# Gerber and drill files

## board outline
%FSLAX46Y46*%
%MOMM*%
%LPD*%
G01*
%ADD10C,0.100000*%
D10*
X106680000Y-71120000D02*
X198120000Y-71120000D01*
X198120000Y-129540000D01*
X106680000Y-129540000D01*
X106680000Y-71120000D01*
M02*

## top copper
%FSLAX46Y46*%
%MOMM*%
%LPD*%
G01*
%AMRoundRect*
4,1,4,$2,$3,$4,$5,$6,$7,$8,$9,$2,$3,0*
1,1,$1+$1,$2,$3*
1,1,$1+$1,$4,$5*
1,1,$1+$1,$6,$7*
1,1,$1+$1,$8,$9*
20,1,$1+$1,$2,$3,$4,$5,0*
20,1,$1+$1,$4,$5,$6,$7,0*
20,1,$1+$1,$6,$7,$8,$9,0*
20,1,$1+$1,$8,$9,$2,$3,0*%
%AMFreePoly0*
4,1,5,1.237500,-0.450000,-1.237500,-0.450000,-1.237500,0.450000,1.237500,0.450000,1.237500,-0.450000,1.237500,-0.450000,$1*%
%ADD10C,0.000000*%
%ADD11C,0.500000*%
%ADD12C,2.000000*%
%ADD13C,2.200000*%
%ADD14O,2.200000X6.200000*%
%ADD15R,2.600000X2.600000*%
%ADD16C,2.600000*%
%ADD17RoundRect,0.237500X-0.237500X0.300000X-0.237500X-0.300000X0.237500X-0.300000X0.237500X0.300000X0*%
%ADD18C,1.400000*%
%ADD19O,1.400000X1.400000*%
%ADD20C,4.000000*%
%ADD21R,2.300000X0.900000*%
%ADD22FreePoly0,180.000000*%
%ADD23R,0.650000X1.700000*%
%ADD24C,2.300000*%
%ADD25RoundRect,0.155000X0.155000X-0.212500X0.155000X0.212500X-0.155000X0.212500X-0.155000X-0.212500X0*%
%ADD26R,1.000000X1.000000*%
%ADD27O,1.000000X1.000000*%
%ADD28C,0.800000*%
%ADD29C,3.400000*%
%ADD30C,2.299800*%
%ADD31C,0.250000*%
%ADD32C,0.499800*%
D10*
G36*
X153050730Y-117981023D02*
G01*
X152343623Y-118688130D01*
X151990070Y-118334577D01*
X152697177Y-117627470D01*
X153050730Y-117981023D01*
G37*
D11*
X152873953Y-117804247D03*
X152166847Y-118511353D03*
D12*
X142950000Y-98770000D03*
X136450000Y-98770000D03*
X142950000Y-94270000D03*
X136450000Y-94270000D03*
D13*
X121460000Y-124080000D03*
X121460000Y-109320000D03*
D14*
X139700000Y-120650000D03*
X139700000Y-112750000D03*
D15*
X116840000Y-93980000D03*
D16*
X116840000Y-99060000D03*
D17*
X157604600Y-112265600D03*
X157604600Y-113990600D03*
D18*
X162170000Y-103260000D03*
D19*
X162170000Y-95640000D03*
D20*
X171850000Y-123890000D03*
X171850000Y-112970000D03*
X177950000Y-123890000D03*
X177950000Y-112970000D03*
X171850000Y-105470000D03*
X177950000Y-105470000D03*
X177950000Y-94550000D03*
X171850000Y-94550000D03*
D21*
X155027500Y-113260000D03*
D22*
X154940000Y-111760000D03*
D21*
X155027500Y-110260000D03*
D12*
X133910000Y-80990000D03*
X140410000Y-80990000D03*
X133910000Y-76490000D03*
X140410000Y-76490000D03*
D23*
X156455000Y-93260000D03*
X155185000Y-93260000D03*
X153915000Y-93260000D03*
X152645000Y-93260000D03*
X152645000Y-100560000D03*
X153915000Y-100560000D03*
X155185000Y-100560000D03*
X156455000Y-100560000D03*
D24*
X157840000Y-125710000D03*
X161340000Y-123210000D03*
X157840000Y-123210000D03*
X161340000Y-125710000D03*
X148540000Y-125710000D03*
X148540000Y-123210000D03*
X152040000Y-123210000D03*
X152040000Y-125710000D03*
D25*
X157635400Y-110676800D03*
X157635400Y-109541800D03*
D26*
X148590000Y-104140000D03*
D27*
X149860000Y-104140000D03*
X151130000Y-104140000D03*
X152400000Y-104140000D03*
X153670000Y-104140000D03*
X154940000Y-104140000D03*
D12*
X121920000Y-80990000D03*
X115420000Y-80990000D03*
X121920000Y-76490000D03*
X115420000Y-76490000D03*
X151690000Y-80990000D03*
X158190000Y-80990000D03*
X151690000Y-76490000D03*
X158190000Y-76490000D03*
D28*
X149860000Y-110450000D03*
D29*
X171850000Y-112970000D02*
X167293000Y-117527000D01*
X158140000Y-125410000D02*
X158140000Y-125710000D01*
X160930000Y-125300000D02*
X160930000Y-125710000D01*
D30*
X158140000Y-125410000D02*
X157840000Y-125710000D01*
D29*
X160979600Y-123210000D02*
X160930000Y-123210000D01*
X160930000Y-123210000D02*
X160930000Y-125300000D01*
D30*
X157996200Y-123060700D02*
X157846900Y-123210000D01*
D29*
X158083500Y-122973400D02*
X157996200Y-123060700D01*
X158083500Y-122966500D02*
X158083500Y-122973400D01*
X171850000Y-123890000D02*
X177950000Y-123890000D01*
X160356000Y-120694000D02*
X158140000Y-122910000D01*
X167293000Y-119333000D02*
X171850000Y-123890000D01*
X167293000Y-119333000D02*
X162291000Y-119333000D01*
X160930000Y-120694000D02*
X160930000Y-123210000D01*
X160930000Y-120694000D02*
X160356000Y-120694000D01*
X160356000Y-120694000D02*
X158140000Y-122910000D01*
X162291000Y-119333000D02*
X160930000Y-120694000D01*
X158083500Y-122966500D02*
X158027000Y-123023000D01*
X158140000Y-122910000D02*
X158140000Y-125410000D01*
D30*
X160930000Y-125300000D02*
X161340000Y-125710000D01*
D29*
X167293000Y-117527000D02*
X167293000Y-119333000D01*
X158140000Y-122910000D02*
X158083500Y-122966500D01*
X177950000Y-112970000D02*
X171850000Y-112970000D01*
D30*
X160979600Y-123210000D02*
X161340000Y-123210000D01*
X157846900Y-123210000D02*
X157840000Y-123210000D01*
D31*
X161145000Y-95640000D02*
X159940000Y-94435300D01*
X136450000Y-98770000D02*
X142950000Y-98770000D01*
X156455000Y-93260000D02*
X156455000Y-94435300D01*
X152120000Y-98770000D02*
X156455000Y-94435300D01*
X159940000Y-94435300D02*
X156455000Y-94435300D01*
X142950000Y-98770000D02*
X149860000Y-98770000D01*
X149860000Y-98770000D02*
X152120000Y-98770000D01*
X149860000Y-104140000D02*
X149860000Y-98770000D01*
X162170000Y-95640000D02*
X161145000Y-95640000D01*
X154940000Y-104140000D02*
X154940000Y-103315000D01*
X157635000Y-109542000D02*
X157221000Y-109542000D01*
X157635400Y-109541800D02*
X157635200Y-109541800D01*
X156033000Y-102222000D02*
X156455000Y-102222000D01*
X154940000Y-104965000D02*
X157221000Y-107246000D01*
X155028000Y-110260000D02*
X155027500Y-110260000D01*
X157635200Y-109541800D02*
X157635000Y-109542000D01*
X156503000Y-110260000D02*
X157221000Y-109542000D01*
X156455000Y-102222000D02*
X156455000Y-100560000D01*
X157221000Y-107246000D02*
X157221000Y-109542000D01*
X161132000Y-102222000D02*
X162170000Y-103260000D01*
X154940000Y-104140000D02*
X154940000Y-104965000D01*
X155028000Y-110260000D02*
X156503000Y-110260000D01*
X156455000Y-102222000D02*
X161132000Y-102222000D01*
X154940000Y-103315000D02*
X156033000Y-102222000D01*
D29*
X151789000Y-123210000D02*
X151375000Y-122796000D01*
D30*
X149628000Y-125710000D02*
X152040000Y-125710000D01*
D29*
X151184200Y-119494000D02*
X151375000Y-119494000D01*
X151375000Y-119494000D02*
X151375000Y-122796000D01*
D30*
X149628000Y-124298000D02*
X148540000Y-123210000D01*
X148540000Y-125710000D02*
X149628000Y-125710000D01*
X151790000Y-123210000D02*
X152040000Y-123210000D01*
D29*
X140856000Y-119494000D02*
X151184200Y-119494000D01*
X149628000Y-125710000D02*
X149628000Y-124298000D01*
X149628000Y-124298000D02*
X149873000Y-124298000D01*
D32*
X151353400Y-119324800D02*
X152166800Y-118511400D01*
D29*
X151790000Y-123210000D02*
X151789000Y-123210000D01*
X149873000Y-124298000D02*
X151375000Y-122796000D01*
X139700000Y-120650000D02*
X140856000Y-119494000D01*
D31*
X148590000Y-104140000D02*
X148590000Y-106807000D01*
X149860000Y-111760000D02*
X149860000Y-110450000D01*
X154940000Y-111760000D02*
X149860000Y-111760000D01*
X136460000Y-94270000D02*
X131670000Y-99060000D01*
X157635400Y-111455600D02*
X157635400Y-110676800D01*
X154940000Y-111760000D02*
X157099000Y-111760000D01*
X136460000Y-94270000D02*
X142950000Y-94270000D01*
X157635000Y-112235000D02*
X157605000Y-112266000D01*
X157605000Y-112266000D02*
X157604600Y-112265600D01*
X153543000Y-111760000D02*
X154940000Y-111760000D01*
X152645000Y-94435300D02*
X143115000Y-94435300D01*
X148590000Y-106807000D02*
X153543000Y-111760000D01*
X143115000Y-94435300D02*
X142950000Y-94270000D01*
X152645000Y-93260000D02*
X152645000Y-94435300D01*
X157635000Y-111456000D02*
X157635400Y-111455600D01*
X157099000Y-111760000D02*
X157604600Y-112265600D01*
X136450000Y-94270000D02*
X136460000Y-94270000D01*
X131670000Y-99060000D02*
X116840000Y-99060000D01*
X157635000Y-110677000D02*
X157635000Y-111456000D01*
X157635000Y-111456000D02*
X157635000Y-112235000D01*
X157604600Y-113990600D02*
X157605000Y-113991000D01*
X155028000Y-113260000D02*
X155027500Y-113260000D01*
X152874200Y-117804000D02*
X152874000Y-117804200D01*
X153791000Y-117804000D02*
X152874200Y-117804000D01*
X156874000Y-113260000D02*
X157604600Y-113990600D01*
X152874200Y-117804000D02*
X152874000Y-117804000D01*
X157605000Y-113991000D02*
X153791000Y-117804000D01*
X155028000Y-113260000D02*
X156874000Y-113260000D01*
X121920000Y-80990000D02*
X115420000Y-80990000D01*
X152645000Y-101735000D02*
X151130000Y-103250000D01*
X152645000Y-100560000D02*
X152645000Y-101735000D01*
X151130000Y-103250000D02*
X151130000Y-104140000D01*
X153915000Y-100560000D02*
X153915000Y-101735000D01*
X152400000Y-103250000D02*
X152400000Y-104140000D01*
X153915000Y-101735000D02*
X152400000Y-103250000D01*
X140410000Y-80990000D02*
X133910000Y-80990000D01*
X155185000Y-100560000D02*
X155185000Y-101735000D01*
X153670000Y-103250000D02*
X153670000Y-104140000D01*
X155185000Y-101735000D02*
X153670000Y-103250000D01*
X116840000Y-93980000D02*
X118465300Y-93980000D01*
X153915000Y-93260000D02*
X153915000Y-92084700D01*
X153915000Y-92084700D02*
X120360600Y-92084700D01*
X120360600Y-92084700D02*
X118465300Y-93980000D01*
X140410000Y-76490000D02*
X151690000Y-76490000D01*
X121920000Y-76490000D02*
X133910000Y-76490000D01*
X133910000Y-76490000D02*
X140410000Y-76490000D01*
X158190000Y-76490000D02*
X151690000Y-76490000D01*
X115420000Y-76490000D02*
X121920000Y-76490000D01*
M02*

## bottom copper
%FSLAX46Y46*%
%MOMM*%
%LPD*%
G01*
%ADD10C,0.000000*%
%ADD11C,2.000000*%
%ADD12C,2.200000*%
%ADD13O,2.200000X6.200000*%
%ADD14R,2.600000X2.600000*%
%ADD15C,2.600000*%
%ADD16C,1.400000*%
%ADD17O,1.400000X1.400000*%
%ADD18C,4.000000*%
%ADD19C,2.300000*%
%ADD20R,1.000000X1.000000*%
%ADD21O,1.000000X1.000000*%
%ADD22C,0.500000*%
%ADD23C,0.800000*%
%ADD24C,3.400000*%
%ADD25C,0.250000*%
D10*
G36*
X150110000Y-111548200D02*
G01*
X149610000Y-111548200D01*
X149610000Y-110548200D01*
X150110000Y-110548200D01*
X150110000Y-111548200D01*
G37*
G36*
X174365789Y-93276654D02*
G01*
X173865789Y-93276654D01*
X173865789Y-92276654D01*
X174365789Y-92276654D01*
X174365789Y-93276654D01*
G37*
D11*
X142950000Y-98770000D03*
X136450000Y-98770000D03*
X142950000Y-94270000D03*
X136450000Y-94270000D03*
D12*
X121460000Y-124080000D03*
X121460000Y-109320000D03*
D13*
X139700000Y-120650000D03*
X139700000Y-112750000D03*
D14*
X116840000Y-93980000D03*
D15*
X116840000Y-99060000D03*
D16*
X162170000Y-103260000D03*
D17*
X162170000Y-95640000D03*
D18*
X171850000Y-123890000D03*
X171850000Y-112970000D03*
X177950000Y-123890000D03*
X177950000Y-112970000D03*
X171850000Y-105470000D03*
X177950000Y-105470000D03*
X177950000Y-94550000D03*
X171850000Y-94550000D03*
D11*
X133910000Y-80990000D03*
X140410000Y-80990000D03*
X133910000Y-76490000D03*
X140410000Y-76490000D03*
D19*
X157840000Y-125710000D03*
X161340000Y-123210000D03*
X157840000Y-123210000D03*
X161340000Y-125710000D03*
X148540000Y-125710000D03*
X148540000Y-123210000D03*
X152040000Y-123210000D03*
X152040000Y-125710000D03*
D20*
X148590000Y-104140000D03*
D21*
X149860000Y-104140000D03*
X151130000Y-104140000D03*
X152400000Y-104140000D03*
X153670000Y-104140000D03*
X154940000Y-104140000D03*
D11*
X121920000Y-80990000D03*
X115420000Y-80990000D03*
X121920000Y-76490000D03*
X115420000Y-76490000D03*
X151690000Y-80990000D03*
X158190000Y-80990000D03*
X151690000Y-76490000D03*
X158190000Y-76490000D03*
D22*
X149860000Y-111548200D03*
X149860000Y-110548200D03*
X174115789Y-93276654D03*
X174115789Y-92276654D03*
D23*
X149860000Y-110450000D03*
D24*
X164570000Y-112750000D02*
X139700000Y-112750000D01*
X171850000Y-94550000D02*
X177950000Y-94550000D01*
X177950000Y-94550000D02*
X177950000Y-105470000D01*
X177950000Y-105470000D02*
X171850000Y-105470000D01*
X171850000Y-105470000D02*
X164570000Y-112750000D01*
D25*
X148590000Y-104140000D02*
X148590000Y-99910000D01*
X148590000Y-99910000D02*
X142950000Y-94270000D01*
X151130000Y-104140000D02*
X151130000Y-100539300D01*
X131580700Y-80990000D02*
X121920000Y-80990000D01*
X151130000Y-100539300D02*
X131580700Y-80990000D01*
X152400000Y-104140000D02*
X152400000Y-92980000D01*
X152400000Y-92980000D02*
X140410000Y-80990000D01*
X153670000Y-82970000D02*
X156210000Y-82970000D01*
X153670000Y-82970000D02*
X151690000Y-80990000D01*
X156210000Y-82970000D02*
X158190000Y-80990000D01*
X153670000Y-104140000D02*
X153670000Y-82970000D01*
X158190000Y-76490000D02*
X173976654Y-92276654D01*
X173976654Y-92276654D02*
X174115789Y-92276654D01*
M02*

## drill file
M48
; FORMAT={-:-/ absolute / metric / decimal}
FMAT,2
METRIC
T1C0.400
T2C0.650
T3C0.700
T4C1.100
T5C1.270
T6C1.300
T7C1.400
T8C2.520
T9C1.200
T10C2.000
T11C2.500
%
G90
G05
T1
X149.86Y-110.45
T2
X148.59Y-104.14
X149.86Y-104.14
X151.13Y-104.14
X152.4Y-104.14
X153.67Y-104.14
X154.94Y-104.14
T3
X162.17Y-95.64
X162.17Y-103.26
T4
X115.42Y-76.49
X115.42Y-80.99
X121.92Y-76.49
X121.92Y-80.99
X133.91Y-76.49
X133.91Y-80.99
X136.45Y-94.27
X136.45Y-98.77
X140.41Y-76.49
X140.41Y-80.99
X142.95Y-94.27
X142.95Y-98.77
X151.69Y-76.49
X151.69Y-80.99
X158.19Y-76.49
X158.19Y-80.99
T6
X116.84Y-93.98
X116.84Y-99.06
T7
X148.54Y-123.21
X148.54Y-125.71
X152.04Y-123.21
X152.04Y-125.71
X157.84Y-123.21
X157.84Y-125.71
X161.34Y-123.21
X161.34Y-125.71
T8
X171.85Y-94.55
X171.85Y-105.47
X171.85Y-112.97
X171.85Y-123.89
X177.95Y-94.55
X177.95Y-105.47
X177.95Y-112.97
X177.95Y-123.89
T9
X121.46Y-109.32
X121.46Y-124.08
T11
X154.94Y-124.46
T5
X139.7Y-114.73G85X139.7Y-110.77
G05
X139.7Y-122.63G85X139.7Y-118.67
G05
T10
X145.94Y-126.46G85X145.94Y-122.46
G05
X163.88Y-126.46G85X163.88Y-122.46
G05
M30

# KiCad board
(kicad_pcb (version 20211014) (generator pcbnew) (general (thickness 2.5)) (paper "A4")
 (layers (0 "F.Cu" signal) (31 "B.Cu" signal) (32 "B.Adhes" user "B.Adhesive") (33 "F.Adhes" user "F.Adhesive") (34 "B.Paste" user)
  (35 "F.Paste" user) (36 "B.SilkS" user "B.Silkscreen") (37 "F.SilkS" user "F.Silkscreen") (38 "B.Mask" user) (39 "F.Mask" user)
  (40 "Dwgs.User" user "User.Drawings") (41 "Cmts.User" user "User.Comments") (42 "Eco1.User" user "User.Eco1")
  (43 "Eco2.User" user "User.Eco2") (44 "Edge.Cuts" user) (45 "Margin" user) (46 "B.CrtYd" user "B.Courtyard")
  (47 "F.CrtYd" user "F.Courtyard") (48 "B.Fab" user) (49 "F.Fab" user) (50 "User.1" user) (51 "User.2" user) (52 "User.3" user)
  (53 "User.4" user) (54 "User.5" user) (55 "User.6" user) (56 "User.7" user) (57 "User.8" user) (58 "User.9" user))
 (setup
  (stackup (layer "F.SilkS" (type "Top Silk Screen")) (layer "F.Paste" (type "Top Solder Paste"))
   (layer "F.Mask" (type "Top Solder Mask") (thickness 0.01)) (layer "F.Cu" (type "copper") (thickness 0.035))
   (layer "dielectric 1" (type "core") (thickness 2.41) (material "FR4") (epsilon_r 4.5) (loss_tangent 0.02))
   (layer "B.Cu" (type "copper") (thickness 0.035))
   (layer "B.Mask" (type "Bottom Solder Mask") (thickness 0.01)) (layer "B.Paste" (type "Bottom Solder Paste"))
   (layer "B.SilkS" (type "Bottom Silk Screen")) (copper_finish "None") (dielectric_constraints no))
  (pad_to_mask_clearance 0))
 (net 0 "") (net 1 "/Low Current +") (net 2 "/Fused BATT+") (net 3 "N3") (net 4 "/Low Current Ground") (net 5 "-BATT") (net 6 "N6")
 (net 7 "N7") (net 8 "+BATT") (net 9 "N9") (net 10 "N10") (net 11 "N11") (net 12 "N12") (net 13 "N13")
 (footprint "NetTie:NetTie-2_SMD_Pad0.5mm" (layer "F.Cu") (at 152.5204 118.1578 -135)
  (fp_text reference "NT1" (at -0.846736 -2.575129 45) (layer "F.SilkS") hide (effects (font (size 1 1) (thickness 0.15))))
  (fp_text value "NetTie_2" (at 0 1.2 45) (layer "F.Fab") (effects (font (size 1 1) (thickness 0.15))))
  (fp_poly (pts (xy -0.5 -0.25) (xy 0.5 -0.25) (xy 0.5 0.25) (xy -0.5 0.25)) (layer "F.Cu") (width 0) (fill solid))
  (pad "1" smd circle (at -0.5 0 225) (size 0.5 0.5) (layers "F.Cu") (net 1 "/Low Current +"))
  (pad "2" smd circle (at 0.5 0 225) (size 0.5 0.5) (layers "F.Cu") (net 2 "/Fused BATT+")))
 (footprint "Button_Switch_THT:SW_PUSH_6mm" (layer "F.Cu") (at 142.95 98.77 180)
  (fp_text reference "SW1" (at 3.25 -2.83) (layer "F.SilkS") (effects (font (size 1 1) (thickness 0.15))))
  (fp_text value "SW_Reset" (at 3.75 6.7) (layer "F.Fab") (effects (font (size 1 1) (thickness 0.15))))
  (pad "1" thru_hole circle (at 0 0 270) (size 2 2) (drill 1.1) (layers *.Cu *.Mask) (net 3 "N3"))
  (pad "1" thru_hole circle (at 6.5 0 270) (size 2 2) (drill 1.1) (layers *.Cu *.Mask) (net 3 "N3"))
  (pad "2" thru_hole circle (at 0 4.5 270) (size 2 2) (drill 1.1) (layers *.Cu *.Mask) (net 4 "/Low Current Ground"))
  (pad "2" thru_hole circle (at 6.5 4.5 270) (size 2 2) (drill 1.1) (layers *.Cu *.Mask) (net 4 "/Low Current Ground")))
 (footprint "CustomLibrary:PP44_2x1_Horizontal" (layer "F.Cu") (at 139.7 120.65 90)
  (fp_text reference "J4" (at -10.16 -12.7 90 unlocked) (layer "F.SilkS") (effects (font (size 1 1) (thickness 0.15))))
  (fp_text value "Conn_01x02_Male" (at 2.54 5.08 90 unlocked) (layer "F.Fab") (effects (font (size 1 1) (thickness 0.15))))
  (pad "" np_thru_hole circle (at -3.43 -18.24 90) (size 2.2 2.2) (drill 1.2) (layers F&B.Cu *.Mask))
  (pad "" np_thru_hole circle (at 11.33 -18.24 90) (size 2.2 2.2) (drill 1.2) (layers F&B.Cu *.Mask))
  (pad "1" thru_hole oval (at 0 0 90) (size 6.2 2.2) (drill oval 5.23 1.27) (layers *.Cu *.Mask) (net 2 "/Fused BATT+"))
  (pad "2" thru_hole oval (at 7.9 0 90) (size 6.2 2.2) (drill oval 5.23 1.27) (layers *.Cu *.Mask) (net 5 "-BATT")))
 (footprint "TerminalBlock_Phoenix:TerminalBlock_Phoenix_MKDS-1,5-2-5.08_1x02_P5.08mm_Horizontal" (layer "F.Cu") (at 116.84 93.98 -90)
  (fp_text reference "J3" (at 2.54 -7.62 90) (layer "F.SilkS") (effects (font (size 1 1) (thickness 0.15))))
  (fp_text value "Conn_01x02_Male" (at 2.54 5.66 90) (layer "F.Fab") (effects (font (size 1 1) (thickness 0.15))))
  (pad "1" thru_hole rect (at 0 0 270) (size 2.6 2.6) (drill 1.3) (layers *.Cu *.Mask) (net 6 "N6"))
  (pad "2" thru_hole circle (at 5.08 0 270) (size 2.6 2.6) (drill 1.3) (layers *.Cu *.Mask) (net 4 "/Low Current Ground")))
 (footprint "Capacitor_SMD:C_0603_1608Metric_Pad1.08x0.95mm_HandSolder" (layer "F.Cu") (at 157.6046 113.1281 -90)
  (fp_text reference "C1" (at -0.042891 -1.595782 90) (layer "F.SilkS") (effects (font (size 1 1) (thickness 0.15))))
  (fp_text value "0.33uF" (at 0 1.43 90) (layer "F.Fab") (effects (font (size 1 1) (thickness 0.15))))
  (pad "1" smd roundrect (at -0.8625 0 270) (size 1.075 0.95) (layers "F.Cu" "F.Paste" "F.Mask") (roundrect_rratio 0.25)
   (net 4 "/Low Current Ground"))
  (pad "2" smd roundrect (at 0.8625 0 270) (size 1.075 0.95) (layers "F.Cu" "F.Paste" "F.Mask") (roundrect_rratio 0.25)
   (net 1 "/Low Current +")))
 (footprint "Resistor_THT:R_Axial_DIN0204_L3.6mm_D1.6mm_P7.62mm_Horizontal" (layer "F.Cu") (at 162.17 103.26 90)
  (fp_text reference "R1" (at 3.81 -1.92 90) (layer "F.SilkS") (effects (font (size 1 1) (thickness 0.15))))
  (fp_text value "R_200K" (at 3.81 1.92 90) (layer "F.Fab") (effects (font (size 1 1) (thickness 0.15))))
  (pad "1" thru_hole circle (at 0 0 90) (size 1.4 1.4) (drill 0.7) (layers *.Cu *.Mask) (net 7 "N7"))
  (pad "2" thru_hole oval (at 7.62 0 90) (size 1.4 1.4) (drill 0.7) (layers *.Cu *.Mask) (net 3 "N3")))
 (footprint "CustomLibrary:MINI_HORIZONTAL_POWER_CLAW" (layer "F.Cu") (at 171.85 123.89)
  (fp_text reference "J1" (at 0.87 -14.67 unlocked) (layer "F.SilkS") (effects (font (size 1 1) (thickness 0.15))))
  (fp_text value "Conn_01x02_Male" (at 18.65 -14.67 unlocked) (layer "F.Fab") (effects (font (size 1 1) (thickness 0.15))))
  (pad "1" thru_hole circle (at 0 0) (size 4 4) (drill 2.52) (layers *.Cu *.Mask) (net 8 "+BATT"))
  (pad "1" thru_hole circle (at 0 -10.92) (size 4 4) (drill 2.52) (layers *.Cu *.Mask) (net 8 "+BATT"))
  (pad "1" thru_hole circle (at 6.1 0) (size 4 4) (drill 2.52) (layers *.Cu *.Mask) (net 8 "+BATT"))
  (pad "1" thru_hole circle (at 6.1 -10.92) (size 4 4) (drill 2.52) (layers *.Cu *.Mask) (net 8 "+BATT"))
  (pad "2" thru_hole circle (at 0 -18.42) (size 4 4) (drill 2.52) (layers *.Cu *.Mask) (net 5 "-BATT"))
  (pad "2" thru_hole circle (at 6.1 -18.42) (size 4 4) (drill 2.52) (layers *.Cu *.Mask) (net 5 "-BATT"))
  (pad "2" thru_hole circle (at 6.1 -29.34) (size 4 4) (drill 2.52) (layers *.Cu *.Mask) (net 5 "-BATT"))
  (pad "2" thru_hole circle (at 0 -29.34) (size 4 4) (drill 2.52) (layers *.Cu *.Mask) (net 5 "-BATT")))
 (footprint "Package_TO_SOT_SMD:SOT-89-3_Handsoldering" (layer "F.Cu") (at 152.8775 111.76 180)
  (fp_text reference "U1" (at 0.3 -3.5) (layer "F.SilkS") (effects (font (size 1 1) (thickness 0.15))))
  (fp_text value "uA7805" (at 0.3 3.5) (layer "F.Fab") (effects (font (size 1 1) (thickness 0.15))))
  (pad "1" smd rect (at -2.15 -1.5 180) (size 2.3 0.9) (layers "F.Cu" "F.Paste" "F.Mask") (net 1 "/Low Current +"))
  (pad "2" smd custom (at -2.0625 0 180) (size 2.475 0.9) (layers "F.Cu" "F.Paste" "F.Mask") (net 4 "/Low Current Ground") (zone_connect 2)
   (options (clearance outline) (anchor rect)) (primitives))
  (pad "3" smd rect (at -2.15 1.5 180) (size 2.3 0.9) (layers "F.Cu" "F.Paste" "F.Mask") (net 7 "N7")))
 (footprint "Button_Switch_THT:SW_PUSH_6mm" (layer "F.Cu") (at 140.41 80.99 180)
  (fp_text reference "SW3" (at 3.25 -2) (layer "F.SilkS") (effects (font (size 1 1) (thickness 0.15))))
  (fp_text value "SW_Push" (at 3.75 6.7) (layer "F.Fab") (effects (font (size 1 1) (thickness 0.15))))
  (pad "1" thru_hole circle (at 6.5 0 270) (size 2 2) (drill 1.1) (layers *.Cu *.Mask) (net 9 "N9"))
  (pad "1" thru_hole circle (at 0 0 270) (size 2 2) (drill 1.1) (layers *.Cu *.Mask) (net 9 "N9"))
  (pad "2" thru_hole circle (at 6.5 4.5 270) (size 2 2) (drill 1.1) (layers *.Cu *.Mask) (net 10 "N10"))
  (pad "2" thru_hole circle (at 0 4.5 270) (size 2 2) (drill 1.1) (layers *.Cu *.Mask) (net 10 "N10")))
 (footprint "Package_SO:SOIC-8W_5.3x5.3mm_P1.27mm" (layer "F.Cu") (at 154.55 96.91 -90)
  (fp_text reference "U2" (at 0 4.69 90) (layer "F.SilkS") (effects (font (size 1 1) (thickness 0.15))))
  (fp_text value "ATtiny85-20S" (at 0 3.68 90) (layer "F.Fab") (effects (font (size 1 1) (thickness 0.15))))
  (pad "1" smd rect (at -3.65 -1.905 270) (size 1.7 0.65) (layers "F.Cu" "F.Paste" "F.Mask") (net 3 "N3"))
  (pad "2" smd rect (at -3.65 -0.635 270) (size 1.7 0.65) (layers "F.Cu" "F.Paste" "F.Mask") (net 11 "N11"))
  (pad "3" smd rect (at -3.65 0.635 270) (size 1.7 0.65) (layers "F.Cu" "F.Paste" "F.Mask") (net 6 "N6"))
  (pad "4" smd rect (at -3.65 1.905 270) (size 1.7 0.65) (layers "F.Cu" "F.Paste" "F.Mask") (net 4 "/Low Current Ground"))
  (pad "5" smd rect (at 3.65 1.905 270) (size 1.7 0.65) (layers "F.Cu" "F.Paste" "F.Mask") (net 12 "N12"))
  (pad "6" smd rect (at 3.65 0.635 270) (size 1.7 0.65) (layers "F.Cu" "F.Paste" "F.Mask") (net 9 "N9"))
  (pad "7" smd rect (at 3.65 -0.635 270) (size 1.7 0.65) (layers "F.Cu" "F.Paste" "F.Mask") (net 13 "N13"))
  (pad "8" smd rect (at 3.65 -1.905 270) (size 1.7 0.65) (layers "F.Cu" "F.Paste" "F.Mask") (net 7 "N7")))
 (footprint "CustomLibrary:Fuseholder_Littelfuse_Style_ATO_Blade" (layer "F.Cu") (at 161.34 125.71 180)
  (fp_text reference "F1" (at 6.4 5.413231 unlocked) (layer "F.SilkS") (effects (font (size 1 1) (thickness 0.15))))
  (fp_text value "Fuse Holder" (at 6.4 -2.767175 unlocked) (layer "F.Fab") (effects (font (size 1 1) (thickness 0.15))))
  (pad "" np_thru_hole circle (at 6.4 1.25 180) (size 2.5 2.5) (drill 2.5) (layers F&B.Cu *.Mask))
  (pad "" np_thru_hole oval (at 15.4 1.25 180) (size 2 6) (drill oval 2 6) (layers F&B.Cu *.Mask))
  (pad "" np_thru_hole oval (at -2.54 1.25 180) (size 2 6) (drill oval 2 6) (layers F&B.Cu *.Mask))
  (pad "1" thru_hole circle (at 3.5 0 180) (size 2.3 2.3) (drill 1.4) (layers *.Cu *.Mask) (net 8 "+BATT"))
  (pad "1" thru_hole circle (at 0 2.5 180) (size 2.3 2.3) (drill 1.4) (layers *.Cu *.Mask) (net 8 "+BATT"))
  (pad "1" thru_hole circle (at 3.5 2.5 180) (size 2.3 2.3) (drill 1.4) (layers *.Cu *.Mask) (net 8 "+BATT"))
  (pad "1" thru_hole circle (at 0 0 180) (size 2.3 2.3) (drill 1.4) (layers *.Cu *.Mask) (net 8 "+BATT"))
  (pad "2" thru_hole circle (at 12.8 0 180) (size 2.3 2.3) (drill 1.4) (layers *.Cu *.Mask) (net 2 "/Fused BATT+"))
  (pad "2" thru_hole circle (at 12.8 2.5 180) (size 2.3 2.3) (drill 1.4) (layers *.Cu *.Mask) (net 2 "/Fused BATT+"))
  (pad "2" thru_hole circle (at 9.3 2.5 180) (size 2.3 2.3) (drill 1.4) (layers *.Cu *.Mask) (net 2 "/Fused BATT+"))
  (pad "2" thru_hole circle (at 9.3 0 180) (size 2.3 2.3) (drill 1.4) (layers *.Cu *.Mask) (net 2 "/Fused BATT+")))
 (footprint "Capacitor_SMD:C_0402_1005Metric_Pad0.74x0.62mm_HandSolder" (layer "F.Cu") (at 157.6354 110.1093 90)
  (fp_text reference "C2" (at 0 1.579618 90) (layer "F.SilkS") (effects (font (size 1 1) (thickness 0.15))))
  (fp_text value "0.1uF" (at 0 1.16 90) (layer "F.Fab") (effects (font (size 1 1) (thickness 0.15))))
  (pad "1" smd roundrect (at -0.5675 0 90) (size 0.735 0.62) (layers "F.Cu" "F.Paste" "F.Mask") (roundrect_rratio 0.25)
   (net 4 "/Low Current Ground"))
  (pad "2" smd roundrect (at 0.5675 0 90) (size 0.735 0.62) (layers "F.Cu" "F.Paste" "F.Mask") (roundrect_rratio 0.25) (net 7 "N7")))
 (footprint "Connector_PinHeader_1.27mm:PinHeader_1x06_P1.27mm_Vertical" (layer "F.Cu") (at 148.59 104.14 90)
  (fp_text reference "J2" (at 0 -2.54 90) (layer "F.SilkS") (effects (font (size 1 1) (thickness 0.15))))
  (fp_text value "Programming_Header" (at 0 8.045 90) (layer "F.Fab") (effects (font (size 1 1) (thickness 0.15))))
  (pad "1" thru_hole rect (at 0 0 90) (size 1 1) (drill 0.65) (layers *.Cu *.Mask) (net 4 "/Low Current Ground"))
  (pad "2" thru_hole oval (at 0 1.27 90) (size 1 1) (drill 0.65) (layers *.Cu *.Mask) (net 3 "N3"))
  (pad "3" thru_hole oval (at 0 2.54 90) (size 1 1) (drill 0.65) (layers *.Cu *.Mask) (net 12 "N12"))
  (pad "4" thru_hole oval (at 0 3.81 90) (size 1 1) (drill 0.65) (layers *.Cu *.Mask) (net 9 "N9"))
  (pad "5" thru_hole oval (at 0 5.08 90) (size 1 1) (drill 0.65) (layers *.Cu *.Mask) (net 13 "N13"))
  (pad "6" thru_hole oval (at 0 6.35 90) (size 1 1) (drill 0.65) (layers *.Cu *.Mask) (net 7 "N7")))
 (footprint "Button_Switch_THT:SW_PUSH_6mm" (layer "F.Cu") (at 121.92 80.99 180)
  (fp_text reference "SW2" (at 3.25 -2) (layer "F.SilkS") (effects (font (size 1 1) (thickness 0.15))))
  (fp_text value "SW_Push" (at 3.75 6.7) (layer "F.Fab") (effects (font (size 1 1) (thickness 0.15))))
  (pad "1" thru_hole circle (at 0 0 270) (size 2 2) (drill 1.1) (layers *.Cu *.Mask) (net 12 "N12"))
  (pad "1" thru_hole circle (at 6.5 0 270) (size 2 2) (drill 1.1) (layers *.Cu *.Mask) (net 12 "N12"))
  (pad "2" thru_hole circle (at 0 4.5 270) (size 2 2) (drill 1.1) (layers *.Cu *.Mask) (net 10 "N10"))
  (pad "2" thru_hole circle (at 6.5 4.5 270) (size 2 2) (drill 1.1) (layers *.Cu *.Mask) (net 10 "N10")))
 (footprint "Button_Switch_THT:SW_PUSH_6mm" (layer "F.Cu") (at 158.19 80.99 180)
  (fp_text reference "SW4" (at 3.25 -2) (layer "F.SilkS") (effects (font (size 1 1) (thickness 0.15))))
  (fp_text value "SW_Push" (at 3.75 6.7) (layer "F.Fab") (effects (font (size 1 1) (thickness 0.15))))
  (pad "1" thru_hole circle (at 6.5 0 270) (size 2 2) (drill 1.1) (layers *.Cu *.Mask) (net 13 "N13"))
  (pad "1" thru_hole circle (at 0 0 270) (size 2 2) (drill 1.1) (layers *.Cu *.Mask) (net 13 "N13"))
  (pad "2" thru_hole circle (at 6.5 4.5 270) (size 2 2) (drill 1.1) (layers *.Cu *.Mask) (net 10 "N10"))
  (pad "2" thru_hole circle (at 0 4.5 270) (size 2 2) (drill 1.1) (layers *.Cu *.Mask) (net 10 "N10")))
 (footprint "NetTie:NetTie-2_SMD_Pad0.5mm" (layer "B.Cu") (at 149.86 111.0482 90)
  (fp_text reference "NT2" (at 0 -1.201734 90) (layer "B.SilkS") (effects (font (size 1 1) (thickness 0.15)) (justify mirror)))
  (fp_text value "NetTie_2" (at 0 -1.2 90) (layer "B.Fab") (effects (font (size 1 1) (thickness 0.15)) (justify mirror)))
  (fp_poly (pts (xy -0.5 0.25) (xy 0.5 0.25) (xy 0.5 -0.25) (xy -0.5 -0.25)) (layer "B.Cu") (width 0) (fill solid))
  (pad "1" smd circle (at -0.5 0 90) (size 0.5 0.5) (layers "B.Cu") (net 5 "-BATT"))
  (pad "2" smd circle (at 0.5 0 90) (size 0.5 0.5) (layers "B.Cu") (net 4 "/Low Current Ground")))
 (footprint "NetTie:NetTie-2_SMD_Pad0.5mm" (layer "B.Cu") (at 174.115789 92.776654 90)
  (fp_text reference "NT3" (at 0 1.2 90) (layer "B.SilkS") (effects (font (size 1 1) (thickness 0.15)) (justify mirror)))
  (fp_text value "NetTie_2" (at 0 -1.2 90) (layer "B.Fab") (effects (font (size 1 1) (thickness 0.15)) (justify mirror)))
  (fp_poly (pts (xy -0.5 0.25) (xy 0.5 0.25) (xy 0.5 -0.25) (xy -0.5 -0.25)) (layer "B.Cu") (width 0) (fill solid))
  (pad "1" smd circle (at -0.5 0 90) (size 0.5 0.5) (layers "B.Cu") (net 5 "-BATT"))
  (pad "2" smd circle (at 0.5 0 90) (size 0.5 0.5) (layers "B.Cu") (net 10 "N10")))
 (gr_rect (start 198.12 129.54) (end 106.68 71.12) (layer "Edge.Cuts") (width 0.1) (fill none))
 (segment (start 171.85 112.97) (end 167.293 117.527) (width 3.4) (layer "F.Cu") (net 8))
 (segment (start 158.14 125.41) (end 158.14 125.71) (width 3.4) (layer "F.Cu") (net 8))
 (segment (start 160.93 125.3) (end 160.93 125.71) (width 3.4) (layer "F.Cu") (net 8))
 (segment (start 158.14 125.41) (end 157.84 125.71) (width 2.2998) (layer "F.Cu") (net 8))
 (segment (start 160.9796 123.21) (end 160.93 123.21) (width 3.4) (layer "F.Cu") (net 8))
 (segment (start 160.93 123.21) (end 160.93 125.3) (width 3.4) (layer "F.Cu") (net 8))
 (segment (start 157.9962 123.0607) (end 157.8469 123.21) (width 2.2998) (layer "F.Cu") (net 8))
 (segment (start 158.0835 122.9734) (end 157.9962 123.0607) (width 3.4) (layer "F.Cu") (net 8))
 (segment (start 158.0835 122.9665) (end 158.0835 122.9734) (width 3.4) (layer "F.Cu") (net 8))
 (segment (start 171.85 123.89) (end 177.95 123.89) (width 3.4) (layer "F.Cu") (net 8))
 (segment (start 160.356 120.694) (end 158.14 122.91) (width 3.4) (layer "F.Cu") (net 8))
 (segment (start 167.293 119.333) (end 171.85 123.89) (width 3.4) (layer "F.Cu") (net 8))
 (segment (start 167.293 119.333) (end 162.291 119.333) (width 3.4) (layer "F.Cu") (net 8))
 (segment (start 160.93 120.694) (end 160.93 123.21) (width 3.4) (layer "F.Cu") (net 8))
 (segment (start 160.93 120.694) (end 160.356 120.694) (width 3.4) (layer "F.Cu") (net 8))
 (segment (start 160.356 120.694) (end 158.14 122.91) (width 3.4) (layer "F.Cu") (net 8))
 (segment (start 162.291 119.333) (end 160.93 120.694) (width 3.4) (layer "F.Cu") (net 8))
 (segment (start 158.0835 122.9665) (end 158.027 123.023) (width 3.4) (layer "F.Cu") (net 8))
 (segment (start 158.14 122.91) (end 158.14 125.41) (width 3.4) (layer "F.Cu") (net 8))
 (segment (start 160.93 125.3) (end 161.34 125.71) (width 2.2998) (layer "F.Cu") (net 8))
 (segment (start 167.293 117.527) (end 167.293 119.333) (width 3.4) (layer "F.Cu") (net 8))
 (segment (start 158.14 122.91) (end 158.0835 122.9665) (width 3.4) (layer "F.Cu") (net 8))
 (segment (start 177.95 112.97) (end 171.85 112.97) (width 3.4) (layer "F.Cu") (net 8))
 (segment (start 160.9796 123.21) (end 161.34 123.21) (width 2.2998) (layer "F.Cu") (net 8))
 (segment (start 157.8469 123.21) (end 157.84 123.21) (width 2.2998) (layer "F.Cu") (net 8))
 (segment (start 164.57 112.75) (end 139.7 112.75) (width 3.4) (layer "B.Cu") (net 5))
 (segment (start 171.85 94.55) (end 177.95 94.55) (width 3.4) (layer "B.Cu") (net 5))
 (segment (start 177.95 94.55) (end 177.95 105.47) (width 3.4) (layer "B.Cu") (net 5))
 (segment (start 177.95 105.47) (end 171.85 105.47) (width 3.4) (layer "B.Cu") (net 5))
 (segment (start 171.85 105.47) (end 164.57 112.75) (width 3.4) (layer "B.Cu") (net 5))
 (segment (start 161.145 95.64) (end 159.94 94.4353) (width 0.25) (layer "F.Cu") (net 3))
 (segment (start 136.45 98.77) (end 142.95 98.77) (width 0.25) (layer "F.Cu") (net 3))
 (segment (start 156.455 93.26) (end 156.455 94.4353) (width 0.25) (layer "F.Cu") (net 3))
 (segment (start 152.12 98.77) (end 156.455 94.4353) (width 0.25) (layer "F.Cu") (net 3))
 (segment (start 159.94 94.4353) (end 156.455 94.4353) (width 0.25) (layer "F.Cu") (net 3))
 (segment (start 142.95 98.77) (end 149.86 98.77) (width 0.25) (layer "F.Cu") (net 3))
 (segment (start 149.86 98.77) (end 152.12 98.77) (width 0.25) (layer "F.Cu") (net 3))
 (segment (start 149.86 104.14) (end 149.86 98.77) (width 0.25) (layer "F.Cu") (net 3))
 (segment (start 162.17 95.64) (end 161.145 95.64) (width 0.25) (layer "F.Cu") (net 3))
 (segment (start 154.94 104.14) (end 154.94 103.315) (width 0.25) (layer "F.Cu") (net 7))
 (segment (start 157.635 109.542) (end 157.221 109.542) (width 0.25) (layer "F.Cu") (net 7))
 (segment (start 157.6354 109.5418) (end 157.6352 109.5418) (width 0.25) (layer "F.Cu") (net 7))
 (segment (start 156.033 102.222) (end 156.455 102.222) (width 0.25) (layer "F.Cu") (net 7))
 (segment (start 154.94 104.965) (end 157.221 107.246) (width 0.25) (layer "F.Cu") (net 7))
 (segment (start 155.028 110.26) (end 155.0275 110.26) (width 0.25) (layer "F.Cu") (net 7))
 (segment (start 157.6352 109.5418) (end 157.635 109.542) (width 0.25) (layer "F.Cu") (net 7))
 (segment (start 156.503 110.26) (end 157.221 109.542) (width 0.25) (layer "F.Cu") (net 7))
 (segment (start 156.455 102.222) (end 156.455 100.56) (width 0.25) (layer "F.Cu") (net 7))
 (segment (start 157.221 107.246) (end 157.221 109.542) (width 0.25) (layer "F.Cu") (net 7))
 (segment (start 161.132 102.222) (end 162.17 103.26) (width 0.25) (layer "F.Cu") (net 7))
 (segment (start 154.94 104.14) (end 154.94 104.965) (width 0.25) (layer "F.Cu") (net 7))
 (segment (start 155.028 110.26) (end 156.503 110.26) (width 0.25) (layer "F.Cu") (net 7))
 (segment (start 156.455 102.222) (end 161.132 102.222) (width 0.25) (layer "F.Cu") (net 7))
 (segment (start 154.94 103.315) (end 156.033 102.222) (width 0.25) (layer "F.Cu") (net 7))
 (segment (start 151.789 123.21) (end 151.375 122.796) (width 3.4) (layer "F.Cu") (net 2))
 (segment (start 149.628 125.71) (end 152.04 125.71) (width 2.2998) (layer "F.Cu") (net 2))
 (segment (start 151.1842 119.494) (end 151.375 119.494) (width 3.4) (layer "F.Cu") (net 2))
 (segment (start 151.375 119.494) (end 151.375 122.796) (width 3.4) (layer "F.Cu") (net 2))
 (segment (start 149.628 124.298) (end 148.54 123.21) (width 2.2998) (layer "F.Cu") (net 2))
 (segment (start 148.54 125.71) (end 149.628 125.71) (width 2.2998) (layer "F.Cu") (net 2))
 (segment (start 151.79 123.21) (end 152.04 123.21) (width 2.2998) (layer "F.Cu") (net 2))
 (segment (start 140.856 119.494) (end 151.1842 119.494) (width 3.4) (layer "F.Cu") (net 2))
 (segment (start 149.628 125.71) (end 149.628 124.298) (width 3.4) (layer "F.Cu") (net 2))
 (segment (start 149.628 124.298) (end 149.873 124.298) (width 3.4) (layer "F.Cu") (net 2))
 (segment (start 151.3534 119.3248) (end 152.1668 118.5114) (width 0.4998) (layer "F.Cu") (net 2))
 (segment (start 151.79 123.21) (end 151.789 123.21) (width 3.4) (layer "F.Cu") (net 2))
 (segment (start 149.873 124.298) (end 151.375 122.796) (width 3.4) (layer "F.Cu") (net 2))
 (segment (start 139.7 120.65) (end 140.856 119.494) (width 3.4) (layer "F.Cu") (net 2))
 (segment (start 148.59 104.14) (end 148.59 106.807) (width 0.25) (layer "F.Cu") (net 4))
 (segment (start 149.86 111.76) (end 149.86 110.45) (width 0.25) (layer "F.Cu") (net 4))
 (segment (start 154.94 111.76) (end 149.86 111.76) (width 0.25) (layer "F.Cu") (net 4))
 (segment (start 136.46 94.27) (end 131.67 99.06) (width 0.25) (layer "F.Cu") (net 4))
 (segment (start 157.6354 111.4556) (end 157.6354 110.6768) (width 0.25) (layer "F.Cu") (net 4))
 (segment (start 154.94 111.76) (end 157.099 111.76) (width 0.25) (layer "F.Cu") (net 4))
 (segment (start 136.46 94.27) (end 142.95 94.27) (width 0.25) (layer "F.Cu") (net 4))
 (segment (start 157.635 112.235) (end 157.605 112.266) (width 0.25) (layer "F.Cu") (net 4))
 (segment (start 157.605 112.266) (end 157.6046 112.2656) (width 0.25) (layer "F.Cu") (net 4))
 (segment (start 153.543 111.76) (end 154.94 111.76) (width 0.25) (layer "F.Cu") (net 4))
 (segment (start 152.645 94.4353) (end 143.115 94.4353) (width 0.25) (layer "F.Cu") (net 4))
 (segment (start 148.59 106.807) (end 153.543 111.76) (width 0.25) (layer "F.Cu") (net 4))
 (segment (start 143.115 94.4353) (end 142.95 94.27) (width 0.25) (layer "F.Cu") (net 4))
 (segment (start 152.645 93.26) (end 152.645 94.4353) (width 0.25) (layer "F.Cu") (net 4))
 (segment (start 157.635 111.456) (end 157.6354 111.4556) (width 0.25) (layer "F.Cu") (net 4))
 (segment (start 157.099 111.76) (end 157.6046 112.2656) (width 0.25) (layer "F.Cu") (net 4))
 (segment (start 136.45 94.27) (end 136.46 94.27) (width 0.25) (layer "F.Cu") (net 4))
 (segment (start 131.67 99.06) (end 116.84 99.06) (width 0.25) (layer "F.Cu") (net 4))
 (segment (start 157.635 110.677) (end 157.635 111.456) (width 0.25) (layer "F.Cu") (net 4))
 (segment (start 157.635 111.456) (end 157.635 112.235) (width 0.25) (layer "F.Cu") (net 4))
 (via (at 149.86 110.45) (size 0.8) (drill 0.4) (layers "F.Cu" "B.Cu") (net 4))
 (segment (start 148.59 104.14) (end 148.59 99.91) (width 0.25) (layer "B.Cu") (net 4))
 (segment (start 148.59 99.91) (end 142.95 94.27) (width 0.25) (layer "B.Cu") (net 4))
 (segment (start 157.6046 113.9906) (end 157.605 113.991) (width 0.25) (layer "F.Cu") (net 1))
 (segment (start 155.028 113.26) (end 155.0275 113.26) (width 0.25) (layer "F.Cu") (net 1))
 (segment (start 152.8742 117.804) (end 152.874 117.8042) (width 0.25) (layer "F.Cu") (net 1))
 (segment (start 153.791 117.804) (end 152.8742 117.804) (width 0.25) (layer "F.Cu") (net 1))
 (segment (start 156.874 113.26) (end 157.6046 113.9906) (width 0.25) (layer "F.Cu") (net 1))
 (segment (start 152.8742 117.804) (end 152.874 117.804) (width 0.25) (layer "F.Cu") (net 1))
 (segment (start 157.605 113.991) (end 153.791 117.804) (width 0.25) (layer "F.Cu") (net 1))
 (segment (start 155.028 113.26) (end 156.874 113.26) (width 0.25) (layer "F.Cu") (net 1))
 (segment (start 121.92 80.99) (end 115.42 80.99) (width 0.25) (layer "F.Cu") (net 12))
 (segment (start 152.645 101.735) (end 151.13 103.25) (width 0.25) (layer "F.Cu") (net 12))
 (segment (start 152.645 100.56) (end 152.645 101.735) (width 0.25) (layer "F.Cu") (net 12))
 (segment (start 151.13 103.25) (end 151.13 104.14) (width 0.25) (layer "F.Cu") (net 12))
 (segment (start 151.13 104.14) (end 151.13 100.5393) (width 0.25) (layer "B.Cu") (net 12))
 (segment (start 131.5807 80.99) (end 121.92 80.99) (width 0.25) (layer "B.Cu") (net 12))
 (segment (start 151.13 100.5393) (end 131.5807 80.99) (width 0.25) (layer "B.Cu") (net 12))
 (segment (start 153.915 100.56) (end 153.915 101.735) (width 0.25) (layer "F.Cu") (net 9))
 (segment (start 152.4 103.25) (end 152.4 104.14) (width 0.25) (layer "F.Cu") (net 9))
 (segment (start 153.915 101.735) (end 152.4 103.25) (width 0.25) (layer "F.Cu") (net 9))
 (segment (start 140.41 80.99) (end 133.91 80.99) (width 0.25) (layer "F.Cu") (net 9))
 (segment (start 152.4 104.14) (end 152.4 92.98) (width 0.25) (layer "B.Cu") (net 9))
 (segment (start 152.4 92.98) (end 140.41 80.99) (width 0.25) (layer "B.Cu") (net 9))
 (segment (start 155.185 100.56) (end 155.185 101.735) (width 0.25) (layer "F.Cu") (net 13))
 (segment (start 153.67 103.25) (end 153.67 104.14) (width 0.25) (layer "F.Cu") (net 13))
 (segment (start 155.185 101.735) (end 153.67 103.25) (width 0.25) (layer "F.Cu") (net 13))
 (segment (start 153.67 82.97) (end 156.21 82.97) (width 0.25) (layer "B.Cu") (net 13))
 (segment (start 153.67 82.97) (end 151.69 80.99) (width 0.25) (layer "B.Cu") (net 13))
 (segment (start 156.21 82.97) (end 158.19 80.99) (width 0.25) (layer "B.Cu") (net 13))
 (segment (start 153.67 104.14) (end 153.67 82.97) (width 0.25) (layer "B.Cu") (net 13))
 (segment (start 116.84 93.98) (end 118.4653 93.98) (width 0.25) (layer "F.Cu") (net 6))
 (segment (start 153.915 93.26) (end 153.915 92.0847) (width 0.25) (layer "F.Cu") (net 6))
 (segment (start 153.915 92.0847) (end 120.3606 92.0847) (width 0.25) (layer "F.Cu") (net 6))
 (segment (start 120.3606 92.0847) (end 118.4653 93.98) (width 0.25) (layer "F.Cu") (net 6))
 (segment (start 140.41 76.49) (end 151.69 76.49) (width 0.25) (layer "F.Cu") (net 10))
 (segment (start 121.92 76.49) (end 133.91 76.49) (width 0.25) (layer "F.Cu") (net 10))
 (segment (start 133.91 76.49) (end 140.41 76.49) (width 0.25) (layer "F.Cu") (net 10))
 (segment (start 158.19 76.49) (end 151.69 76.49) (width 0.25) (layer "F.Cu") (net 10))
 (segment (start 115.42 76.49) (end 121.92 76.49) (width 0.25) (layer "F.Cu") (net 10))
 (segment (start 158.19 76.49) (end 173.976654 92.276654) (width 0.25) (layer "B.Cu") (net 10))
 (segment (start 173.976654 92.276654) (end 174.115789 92.276654) (width 0.25) (layer "B.Cu") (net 10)))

